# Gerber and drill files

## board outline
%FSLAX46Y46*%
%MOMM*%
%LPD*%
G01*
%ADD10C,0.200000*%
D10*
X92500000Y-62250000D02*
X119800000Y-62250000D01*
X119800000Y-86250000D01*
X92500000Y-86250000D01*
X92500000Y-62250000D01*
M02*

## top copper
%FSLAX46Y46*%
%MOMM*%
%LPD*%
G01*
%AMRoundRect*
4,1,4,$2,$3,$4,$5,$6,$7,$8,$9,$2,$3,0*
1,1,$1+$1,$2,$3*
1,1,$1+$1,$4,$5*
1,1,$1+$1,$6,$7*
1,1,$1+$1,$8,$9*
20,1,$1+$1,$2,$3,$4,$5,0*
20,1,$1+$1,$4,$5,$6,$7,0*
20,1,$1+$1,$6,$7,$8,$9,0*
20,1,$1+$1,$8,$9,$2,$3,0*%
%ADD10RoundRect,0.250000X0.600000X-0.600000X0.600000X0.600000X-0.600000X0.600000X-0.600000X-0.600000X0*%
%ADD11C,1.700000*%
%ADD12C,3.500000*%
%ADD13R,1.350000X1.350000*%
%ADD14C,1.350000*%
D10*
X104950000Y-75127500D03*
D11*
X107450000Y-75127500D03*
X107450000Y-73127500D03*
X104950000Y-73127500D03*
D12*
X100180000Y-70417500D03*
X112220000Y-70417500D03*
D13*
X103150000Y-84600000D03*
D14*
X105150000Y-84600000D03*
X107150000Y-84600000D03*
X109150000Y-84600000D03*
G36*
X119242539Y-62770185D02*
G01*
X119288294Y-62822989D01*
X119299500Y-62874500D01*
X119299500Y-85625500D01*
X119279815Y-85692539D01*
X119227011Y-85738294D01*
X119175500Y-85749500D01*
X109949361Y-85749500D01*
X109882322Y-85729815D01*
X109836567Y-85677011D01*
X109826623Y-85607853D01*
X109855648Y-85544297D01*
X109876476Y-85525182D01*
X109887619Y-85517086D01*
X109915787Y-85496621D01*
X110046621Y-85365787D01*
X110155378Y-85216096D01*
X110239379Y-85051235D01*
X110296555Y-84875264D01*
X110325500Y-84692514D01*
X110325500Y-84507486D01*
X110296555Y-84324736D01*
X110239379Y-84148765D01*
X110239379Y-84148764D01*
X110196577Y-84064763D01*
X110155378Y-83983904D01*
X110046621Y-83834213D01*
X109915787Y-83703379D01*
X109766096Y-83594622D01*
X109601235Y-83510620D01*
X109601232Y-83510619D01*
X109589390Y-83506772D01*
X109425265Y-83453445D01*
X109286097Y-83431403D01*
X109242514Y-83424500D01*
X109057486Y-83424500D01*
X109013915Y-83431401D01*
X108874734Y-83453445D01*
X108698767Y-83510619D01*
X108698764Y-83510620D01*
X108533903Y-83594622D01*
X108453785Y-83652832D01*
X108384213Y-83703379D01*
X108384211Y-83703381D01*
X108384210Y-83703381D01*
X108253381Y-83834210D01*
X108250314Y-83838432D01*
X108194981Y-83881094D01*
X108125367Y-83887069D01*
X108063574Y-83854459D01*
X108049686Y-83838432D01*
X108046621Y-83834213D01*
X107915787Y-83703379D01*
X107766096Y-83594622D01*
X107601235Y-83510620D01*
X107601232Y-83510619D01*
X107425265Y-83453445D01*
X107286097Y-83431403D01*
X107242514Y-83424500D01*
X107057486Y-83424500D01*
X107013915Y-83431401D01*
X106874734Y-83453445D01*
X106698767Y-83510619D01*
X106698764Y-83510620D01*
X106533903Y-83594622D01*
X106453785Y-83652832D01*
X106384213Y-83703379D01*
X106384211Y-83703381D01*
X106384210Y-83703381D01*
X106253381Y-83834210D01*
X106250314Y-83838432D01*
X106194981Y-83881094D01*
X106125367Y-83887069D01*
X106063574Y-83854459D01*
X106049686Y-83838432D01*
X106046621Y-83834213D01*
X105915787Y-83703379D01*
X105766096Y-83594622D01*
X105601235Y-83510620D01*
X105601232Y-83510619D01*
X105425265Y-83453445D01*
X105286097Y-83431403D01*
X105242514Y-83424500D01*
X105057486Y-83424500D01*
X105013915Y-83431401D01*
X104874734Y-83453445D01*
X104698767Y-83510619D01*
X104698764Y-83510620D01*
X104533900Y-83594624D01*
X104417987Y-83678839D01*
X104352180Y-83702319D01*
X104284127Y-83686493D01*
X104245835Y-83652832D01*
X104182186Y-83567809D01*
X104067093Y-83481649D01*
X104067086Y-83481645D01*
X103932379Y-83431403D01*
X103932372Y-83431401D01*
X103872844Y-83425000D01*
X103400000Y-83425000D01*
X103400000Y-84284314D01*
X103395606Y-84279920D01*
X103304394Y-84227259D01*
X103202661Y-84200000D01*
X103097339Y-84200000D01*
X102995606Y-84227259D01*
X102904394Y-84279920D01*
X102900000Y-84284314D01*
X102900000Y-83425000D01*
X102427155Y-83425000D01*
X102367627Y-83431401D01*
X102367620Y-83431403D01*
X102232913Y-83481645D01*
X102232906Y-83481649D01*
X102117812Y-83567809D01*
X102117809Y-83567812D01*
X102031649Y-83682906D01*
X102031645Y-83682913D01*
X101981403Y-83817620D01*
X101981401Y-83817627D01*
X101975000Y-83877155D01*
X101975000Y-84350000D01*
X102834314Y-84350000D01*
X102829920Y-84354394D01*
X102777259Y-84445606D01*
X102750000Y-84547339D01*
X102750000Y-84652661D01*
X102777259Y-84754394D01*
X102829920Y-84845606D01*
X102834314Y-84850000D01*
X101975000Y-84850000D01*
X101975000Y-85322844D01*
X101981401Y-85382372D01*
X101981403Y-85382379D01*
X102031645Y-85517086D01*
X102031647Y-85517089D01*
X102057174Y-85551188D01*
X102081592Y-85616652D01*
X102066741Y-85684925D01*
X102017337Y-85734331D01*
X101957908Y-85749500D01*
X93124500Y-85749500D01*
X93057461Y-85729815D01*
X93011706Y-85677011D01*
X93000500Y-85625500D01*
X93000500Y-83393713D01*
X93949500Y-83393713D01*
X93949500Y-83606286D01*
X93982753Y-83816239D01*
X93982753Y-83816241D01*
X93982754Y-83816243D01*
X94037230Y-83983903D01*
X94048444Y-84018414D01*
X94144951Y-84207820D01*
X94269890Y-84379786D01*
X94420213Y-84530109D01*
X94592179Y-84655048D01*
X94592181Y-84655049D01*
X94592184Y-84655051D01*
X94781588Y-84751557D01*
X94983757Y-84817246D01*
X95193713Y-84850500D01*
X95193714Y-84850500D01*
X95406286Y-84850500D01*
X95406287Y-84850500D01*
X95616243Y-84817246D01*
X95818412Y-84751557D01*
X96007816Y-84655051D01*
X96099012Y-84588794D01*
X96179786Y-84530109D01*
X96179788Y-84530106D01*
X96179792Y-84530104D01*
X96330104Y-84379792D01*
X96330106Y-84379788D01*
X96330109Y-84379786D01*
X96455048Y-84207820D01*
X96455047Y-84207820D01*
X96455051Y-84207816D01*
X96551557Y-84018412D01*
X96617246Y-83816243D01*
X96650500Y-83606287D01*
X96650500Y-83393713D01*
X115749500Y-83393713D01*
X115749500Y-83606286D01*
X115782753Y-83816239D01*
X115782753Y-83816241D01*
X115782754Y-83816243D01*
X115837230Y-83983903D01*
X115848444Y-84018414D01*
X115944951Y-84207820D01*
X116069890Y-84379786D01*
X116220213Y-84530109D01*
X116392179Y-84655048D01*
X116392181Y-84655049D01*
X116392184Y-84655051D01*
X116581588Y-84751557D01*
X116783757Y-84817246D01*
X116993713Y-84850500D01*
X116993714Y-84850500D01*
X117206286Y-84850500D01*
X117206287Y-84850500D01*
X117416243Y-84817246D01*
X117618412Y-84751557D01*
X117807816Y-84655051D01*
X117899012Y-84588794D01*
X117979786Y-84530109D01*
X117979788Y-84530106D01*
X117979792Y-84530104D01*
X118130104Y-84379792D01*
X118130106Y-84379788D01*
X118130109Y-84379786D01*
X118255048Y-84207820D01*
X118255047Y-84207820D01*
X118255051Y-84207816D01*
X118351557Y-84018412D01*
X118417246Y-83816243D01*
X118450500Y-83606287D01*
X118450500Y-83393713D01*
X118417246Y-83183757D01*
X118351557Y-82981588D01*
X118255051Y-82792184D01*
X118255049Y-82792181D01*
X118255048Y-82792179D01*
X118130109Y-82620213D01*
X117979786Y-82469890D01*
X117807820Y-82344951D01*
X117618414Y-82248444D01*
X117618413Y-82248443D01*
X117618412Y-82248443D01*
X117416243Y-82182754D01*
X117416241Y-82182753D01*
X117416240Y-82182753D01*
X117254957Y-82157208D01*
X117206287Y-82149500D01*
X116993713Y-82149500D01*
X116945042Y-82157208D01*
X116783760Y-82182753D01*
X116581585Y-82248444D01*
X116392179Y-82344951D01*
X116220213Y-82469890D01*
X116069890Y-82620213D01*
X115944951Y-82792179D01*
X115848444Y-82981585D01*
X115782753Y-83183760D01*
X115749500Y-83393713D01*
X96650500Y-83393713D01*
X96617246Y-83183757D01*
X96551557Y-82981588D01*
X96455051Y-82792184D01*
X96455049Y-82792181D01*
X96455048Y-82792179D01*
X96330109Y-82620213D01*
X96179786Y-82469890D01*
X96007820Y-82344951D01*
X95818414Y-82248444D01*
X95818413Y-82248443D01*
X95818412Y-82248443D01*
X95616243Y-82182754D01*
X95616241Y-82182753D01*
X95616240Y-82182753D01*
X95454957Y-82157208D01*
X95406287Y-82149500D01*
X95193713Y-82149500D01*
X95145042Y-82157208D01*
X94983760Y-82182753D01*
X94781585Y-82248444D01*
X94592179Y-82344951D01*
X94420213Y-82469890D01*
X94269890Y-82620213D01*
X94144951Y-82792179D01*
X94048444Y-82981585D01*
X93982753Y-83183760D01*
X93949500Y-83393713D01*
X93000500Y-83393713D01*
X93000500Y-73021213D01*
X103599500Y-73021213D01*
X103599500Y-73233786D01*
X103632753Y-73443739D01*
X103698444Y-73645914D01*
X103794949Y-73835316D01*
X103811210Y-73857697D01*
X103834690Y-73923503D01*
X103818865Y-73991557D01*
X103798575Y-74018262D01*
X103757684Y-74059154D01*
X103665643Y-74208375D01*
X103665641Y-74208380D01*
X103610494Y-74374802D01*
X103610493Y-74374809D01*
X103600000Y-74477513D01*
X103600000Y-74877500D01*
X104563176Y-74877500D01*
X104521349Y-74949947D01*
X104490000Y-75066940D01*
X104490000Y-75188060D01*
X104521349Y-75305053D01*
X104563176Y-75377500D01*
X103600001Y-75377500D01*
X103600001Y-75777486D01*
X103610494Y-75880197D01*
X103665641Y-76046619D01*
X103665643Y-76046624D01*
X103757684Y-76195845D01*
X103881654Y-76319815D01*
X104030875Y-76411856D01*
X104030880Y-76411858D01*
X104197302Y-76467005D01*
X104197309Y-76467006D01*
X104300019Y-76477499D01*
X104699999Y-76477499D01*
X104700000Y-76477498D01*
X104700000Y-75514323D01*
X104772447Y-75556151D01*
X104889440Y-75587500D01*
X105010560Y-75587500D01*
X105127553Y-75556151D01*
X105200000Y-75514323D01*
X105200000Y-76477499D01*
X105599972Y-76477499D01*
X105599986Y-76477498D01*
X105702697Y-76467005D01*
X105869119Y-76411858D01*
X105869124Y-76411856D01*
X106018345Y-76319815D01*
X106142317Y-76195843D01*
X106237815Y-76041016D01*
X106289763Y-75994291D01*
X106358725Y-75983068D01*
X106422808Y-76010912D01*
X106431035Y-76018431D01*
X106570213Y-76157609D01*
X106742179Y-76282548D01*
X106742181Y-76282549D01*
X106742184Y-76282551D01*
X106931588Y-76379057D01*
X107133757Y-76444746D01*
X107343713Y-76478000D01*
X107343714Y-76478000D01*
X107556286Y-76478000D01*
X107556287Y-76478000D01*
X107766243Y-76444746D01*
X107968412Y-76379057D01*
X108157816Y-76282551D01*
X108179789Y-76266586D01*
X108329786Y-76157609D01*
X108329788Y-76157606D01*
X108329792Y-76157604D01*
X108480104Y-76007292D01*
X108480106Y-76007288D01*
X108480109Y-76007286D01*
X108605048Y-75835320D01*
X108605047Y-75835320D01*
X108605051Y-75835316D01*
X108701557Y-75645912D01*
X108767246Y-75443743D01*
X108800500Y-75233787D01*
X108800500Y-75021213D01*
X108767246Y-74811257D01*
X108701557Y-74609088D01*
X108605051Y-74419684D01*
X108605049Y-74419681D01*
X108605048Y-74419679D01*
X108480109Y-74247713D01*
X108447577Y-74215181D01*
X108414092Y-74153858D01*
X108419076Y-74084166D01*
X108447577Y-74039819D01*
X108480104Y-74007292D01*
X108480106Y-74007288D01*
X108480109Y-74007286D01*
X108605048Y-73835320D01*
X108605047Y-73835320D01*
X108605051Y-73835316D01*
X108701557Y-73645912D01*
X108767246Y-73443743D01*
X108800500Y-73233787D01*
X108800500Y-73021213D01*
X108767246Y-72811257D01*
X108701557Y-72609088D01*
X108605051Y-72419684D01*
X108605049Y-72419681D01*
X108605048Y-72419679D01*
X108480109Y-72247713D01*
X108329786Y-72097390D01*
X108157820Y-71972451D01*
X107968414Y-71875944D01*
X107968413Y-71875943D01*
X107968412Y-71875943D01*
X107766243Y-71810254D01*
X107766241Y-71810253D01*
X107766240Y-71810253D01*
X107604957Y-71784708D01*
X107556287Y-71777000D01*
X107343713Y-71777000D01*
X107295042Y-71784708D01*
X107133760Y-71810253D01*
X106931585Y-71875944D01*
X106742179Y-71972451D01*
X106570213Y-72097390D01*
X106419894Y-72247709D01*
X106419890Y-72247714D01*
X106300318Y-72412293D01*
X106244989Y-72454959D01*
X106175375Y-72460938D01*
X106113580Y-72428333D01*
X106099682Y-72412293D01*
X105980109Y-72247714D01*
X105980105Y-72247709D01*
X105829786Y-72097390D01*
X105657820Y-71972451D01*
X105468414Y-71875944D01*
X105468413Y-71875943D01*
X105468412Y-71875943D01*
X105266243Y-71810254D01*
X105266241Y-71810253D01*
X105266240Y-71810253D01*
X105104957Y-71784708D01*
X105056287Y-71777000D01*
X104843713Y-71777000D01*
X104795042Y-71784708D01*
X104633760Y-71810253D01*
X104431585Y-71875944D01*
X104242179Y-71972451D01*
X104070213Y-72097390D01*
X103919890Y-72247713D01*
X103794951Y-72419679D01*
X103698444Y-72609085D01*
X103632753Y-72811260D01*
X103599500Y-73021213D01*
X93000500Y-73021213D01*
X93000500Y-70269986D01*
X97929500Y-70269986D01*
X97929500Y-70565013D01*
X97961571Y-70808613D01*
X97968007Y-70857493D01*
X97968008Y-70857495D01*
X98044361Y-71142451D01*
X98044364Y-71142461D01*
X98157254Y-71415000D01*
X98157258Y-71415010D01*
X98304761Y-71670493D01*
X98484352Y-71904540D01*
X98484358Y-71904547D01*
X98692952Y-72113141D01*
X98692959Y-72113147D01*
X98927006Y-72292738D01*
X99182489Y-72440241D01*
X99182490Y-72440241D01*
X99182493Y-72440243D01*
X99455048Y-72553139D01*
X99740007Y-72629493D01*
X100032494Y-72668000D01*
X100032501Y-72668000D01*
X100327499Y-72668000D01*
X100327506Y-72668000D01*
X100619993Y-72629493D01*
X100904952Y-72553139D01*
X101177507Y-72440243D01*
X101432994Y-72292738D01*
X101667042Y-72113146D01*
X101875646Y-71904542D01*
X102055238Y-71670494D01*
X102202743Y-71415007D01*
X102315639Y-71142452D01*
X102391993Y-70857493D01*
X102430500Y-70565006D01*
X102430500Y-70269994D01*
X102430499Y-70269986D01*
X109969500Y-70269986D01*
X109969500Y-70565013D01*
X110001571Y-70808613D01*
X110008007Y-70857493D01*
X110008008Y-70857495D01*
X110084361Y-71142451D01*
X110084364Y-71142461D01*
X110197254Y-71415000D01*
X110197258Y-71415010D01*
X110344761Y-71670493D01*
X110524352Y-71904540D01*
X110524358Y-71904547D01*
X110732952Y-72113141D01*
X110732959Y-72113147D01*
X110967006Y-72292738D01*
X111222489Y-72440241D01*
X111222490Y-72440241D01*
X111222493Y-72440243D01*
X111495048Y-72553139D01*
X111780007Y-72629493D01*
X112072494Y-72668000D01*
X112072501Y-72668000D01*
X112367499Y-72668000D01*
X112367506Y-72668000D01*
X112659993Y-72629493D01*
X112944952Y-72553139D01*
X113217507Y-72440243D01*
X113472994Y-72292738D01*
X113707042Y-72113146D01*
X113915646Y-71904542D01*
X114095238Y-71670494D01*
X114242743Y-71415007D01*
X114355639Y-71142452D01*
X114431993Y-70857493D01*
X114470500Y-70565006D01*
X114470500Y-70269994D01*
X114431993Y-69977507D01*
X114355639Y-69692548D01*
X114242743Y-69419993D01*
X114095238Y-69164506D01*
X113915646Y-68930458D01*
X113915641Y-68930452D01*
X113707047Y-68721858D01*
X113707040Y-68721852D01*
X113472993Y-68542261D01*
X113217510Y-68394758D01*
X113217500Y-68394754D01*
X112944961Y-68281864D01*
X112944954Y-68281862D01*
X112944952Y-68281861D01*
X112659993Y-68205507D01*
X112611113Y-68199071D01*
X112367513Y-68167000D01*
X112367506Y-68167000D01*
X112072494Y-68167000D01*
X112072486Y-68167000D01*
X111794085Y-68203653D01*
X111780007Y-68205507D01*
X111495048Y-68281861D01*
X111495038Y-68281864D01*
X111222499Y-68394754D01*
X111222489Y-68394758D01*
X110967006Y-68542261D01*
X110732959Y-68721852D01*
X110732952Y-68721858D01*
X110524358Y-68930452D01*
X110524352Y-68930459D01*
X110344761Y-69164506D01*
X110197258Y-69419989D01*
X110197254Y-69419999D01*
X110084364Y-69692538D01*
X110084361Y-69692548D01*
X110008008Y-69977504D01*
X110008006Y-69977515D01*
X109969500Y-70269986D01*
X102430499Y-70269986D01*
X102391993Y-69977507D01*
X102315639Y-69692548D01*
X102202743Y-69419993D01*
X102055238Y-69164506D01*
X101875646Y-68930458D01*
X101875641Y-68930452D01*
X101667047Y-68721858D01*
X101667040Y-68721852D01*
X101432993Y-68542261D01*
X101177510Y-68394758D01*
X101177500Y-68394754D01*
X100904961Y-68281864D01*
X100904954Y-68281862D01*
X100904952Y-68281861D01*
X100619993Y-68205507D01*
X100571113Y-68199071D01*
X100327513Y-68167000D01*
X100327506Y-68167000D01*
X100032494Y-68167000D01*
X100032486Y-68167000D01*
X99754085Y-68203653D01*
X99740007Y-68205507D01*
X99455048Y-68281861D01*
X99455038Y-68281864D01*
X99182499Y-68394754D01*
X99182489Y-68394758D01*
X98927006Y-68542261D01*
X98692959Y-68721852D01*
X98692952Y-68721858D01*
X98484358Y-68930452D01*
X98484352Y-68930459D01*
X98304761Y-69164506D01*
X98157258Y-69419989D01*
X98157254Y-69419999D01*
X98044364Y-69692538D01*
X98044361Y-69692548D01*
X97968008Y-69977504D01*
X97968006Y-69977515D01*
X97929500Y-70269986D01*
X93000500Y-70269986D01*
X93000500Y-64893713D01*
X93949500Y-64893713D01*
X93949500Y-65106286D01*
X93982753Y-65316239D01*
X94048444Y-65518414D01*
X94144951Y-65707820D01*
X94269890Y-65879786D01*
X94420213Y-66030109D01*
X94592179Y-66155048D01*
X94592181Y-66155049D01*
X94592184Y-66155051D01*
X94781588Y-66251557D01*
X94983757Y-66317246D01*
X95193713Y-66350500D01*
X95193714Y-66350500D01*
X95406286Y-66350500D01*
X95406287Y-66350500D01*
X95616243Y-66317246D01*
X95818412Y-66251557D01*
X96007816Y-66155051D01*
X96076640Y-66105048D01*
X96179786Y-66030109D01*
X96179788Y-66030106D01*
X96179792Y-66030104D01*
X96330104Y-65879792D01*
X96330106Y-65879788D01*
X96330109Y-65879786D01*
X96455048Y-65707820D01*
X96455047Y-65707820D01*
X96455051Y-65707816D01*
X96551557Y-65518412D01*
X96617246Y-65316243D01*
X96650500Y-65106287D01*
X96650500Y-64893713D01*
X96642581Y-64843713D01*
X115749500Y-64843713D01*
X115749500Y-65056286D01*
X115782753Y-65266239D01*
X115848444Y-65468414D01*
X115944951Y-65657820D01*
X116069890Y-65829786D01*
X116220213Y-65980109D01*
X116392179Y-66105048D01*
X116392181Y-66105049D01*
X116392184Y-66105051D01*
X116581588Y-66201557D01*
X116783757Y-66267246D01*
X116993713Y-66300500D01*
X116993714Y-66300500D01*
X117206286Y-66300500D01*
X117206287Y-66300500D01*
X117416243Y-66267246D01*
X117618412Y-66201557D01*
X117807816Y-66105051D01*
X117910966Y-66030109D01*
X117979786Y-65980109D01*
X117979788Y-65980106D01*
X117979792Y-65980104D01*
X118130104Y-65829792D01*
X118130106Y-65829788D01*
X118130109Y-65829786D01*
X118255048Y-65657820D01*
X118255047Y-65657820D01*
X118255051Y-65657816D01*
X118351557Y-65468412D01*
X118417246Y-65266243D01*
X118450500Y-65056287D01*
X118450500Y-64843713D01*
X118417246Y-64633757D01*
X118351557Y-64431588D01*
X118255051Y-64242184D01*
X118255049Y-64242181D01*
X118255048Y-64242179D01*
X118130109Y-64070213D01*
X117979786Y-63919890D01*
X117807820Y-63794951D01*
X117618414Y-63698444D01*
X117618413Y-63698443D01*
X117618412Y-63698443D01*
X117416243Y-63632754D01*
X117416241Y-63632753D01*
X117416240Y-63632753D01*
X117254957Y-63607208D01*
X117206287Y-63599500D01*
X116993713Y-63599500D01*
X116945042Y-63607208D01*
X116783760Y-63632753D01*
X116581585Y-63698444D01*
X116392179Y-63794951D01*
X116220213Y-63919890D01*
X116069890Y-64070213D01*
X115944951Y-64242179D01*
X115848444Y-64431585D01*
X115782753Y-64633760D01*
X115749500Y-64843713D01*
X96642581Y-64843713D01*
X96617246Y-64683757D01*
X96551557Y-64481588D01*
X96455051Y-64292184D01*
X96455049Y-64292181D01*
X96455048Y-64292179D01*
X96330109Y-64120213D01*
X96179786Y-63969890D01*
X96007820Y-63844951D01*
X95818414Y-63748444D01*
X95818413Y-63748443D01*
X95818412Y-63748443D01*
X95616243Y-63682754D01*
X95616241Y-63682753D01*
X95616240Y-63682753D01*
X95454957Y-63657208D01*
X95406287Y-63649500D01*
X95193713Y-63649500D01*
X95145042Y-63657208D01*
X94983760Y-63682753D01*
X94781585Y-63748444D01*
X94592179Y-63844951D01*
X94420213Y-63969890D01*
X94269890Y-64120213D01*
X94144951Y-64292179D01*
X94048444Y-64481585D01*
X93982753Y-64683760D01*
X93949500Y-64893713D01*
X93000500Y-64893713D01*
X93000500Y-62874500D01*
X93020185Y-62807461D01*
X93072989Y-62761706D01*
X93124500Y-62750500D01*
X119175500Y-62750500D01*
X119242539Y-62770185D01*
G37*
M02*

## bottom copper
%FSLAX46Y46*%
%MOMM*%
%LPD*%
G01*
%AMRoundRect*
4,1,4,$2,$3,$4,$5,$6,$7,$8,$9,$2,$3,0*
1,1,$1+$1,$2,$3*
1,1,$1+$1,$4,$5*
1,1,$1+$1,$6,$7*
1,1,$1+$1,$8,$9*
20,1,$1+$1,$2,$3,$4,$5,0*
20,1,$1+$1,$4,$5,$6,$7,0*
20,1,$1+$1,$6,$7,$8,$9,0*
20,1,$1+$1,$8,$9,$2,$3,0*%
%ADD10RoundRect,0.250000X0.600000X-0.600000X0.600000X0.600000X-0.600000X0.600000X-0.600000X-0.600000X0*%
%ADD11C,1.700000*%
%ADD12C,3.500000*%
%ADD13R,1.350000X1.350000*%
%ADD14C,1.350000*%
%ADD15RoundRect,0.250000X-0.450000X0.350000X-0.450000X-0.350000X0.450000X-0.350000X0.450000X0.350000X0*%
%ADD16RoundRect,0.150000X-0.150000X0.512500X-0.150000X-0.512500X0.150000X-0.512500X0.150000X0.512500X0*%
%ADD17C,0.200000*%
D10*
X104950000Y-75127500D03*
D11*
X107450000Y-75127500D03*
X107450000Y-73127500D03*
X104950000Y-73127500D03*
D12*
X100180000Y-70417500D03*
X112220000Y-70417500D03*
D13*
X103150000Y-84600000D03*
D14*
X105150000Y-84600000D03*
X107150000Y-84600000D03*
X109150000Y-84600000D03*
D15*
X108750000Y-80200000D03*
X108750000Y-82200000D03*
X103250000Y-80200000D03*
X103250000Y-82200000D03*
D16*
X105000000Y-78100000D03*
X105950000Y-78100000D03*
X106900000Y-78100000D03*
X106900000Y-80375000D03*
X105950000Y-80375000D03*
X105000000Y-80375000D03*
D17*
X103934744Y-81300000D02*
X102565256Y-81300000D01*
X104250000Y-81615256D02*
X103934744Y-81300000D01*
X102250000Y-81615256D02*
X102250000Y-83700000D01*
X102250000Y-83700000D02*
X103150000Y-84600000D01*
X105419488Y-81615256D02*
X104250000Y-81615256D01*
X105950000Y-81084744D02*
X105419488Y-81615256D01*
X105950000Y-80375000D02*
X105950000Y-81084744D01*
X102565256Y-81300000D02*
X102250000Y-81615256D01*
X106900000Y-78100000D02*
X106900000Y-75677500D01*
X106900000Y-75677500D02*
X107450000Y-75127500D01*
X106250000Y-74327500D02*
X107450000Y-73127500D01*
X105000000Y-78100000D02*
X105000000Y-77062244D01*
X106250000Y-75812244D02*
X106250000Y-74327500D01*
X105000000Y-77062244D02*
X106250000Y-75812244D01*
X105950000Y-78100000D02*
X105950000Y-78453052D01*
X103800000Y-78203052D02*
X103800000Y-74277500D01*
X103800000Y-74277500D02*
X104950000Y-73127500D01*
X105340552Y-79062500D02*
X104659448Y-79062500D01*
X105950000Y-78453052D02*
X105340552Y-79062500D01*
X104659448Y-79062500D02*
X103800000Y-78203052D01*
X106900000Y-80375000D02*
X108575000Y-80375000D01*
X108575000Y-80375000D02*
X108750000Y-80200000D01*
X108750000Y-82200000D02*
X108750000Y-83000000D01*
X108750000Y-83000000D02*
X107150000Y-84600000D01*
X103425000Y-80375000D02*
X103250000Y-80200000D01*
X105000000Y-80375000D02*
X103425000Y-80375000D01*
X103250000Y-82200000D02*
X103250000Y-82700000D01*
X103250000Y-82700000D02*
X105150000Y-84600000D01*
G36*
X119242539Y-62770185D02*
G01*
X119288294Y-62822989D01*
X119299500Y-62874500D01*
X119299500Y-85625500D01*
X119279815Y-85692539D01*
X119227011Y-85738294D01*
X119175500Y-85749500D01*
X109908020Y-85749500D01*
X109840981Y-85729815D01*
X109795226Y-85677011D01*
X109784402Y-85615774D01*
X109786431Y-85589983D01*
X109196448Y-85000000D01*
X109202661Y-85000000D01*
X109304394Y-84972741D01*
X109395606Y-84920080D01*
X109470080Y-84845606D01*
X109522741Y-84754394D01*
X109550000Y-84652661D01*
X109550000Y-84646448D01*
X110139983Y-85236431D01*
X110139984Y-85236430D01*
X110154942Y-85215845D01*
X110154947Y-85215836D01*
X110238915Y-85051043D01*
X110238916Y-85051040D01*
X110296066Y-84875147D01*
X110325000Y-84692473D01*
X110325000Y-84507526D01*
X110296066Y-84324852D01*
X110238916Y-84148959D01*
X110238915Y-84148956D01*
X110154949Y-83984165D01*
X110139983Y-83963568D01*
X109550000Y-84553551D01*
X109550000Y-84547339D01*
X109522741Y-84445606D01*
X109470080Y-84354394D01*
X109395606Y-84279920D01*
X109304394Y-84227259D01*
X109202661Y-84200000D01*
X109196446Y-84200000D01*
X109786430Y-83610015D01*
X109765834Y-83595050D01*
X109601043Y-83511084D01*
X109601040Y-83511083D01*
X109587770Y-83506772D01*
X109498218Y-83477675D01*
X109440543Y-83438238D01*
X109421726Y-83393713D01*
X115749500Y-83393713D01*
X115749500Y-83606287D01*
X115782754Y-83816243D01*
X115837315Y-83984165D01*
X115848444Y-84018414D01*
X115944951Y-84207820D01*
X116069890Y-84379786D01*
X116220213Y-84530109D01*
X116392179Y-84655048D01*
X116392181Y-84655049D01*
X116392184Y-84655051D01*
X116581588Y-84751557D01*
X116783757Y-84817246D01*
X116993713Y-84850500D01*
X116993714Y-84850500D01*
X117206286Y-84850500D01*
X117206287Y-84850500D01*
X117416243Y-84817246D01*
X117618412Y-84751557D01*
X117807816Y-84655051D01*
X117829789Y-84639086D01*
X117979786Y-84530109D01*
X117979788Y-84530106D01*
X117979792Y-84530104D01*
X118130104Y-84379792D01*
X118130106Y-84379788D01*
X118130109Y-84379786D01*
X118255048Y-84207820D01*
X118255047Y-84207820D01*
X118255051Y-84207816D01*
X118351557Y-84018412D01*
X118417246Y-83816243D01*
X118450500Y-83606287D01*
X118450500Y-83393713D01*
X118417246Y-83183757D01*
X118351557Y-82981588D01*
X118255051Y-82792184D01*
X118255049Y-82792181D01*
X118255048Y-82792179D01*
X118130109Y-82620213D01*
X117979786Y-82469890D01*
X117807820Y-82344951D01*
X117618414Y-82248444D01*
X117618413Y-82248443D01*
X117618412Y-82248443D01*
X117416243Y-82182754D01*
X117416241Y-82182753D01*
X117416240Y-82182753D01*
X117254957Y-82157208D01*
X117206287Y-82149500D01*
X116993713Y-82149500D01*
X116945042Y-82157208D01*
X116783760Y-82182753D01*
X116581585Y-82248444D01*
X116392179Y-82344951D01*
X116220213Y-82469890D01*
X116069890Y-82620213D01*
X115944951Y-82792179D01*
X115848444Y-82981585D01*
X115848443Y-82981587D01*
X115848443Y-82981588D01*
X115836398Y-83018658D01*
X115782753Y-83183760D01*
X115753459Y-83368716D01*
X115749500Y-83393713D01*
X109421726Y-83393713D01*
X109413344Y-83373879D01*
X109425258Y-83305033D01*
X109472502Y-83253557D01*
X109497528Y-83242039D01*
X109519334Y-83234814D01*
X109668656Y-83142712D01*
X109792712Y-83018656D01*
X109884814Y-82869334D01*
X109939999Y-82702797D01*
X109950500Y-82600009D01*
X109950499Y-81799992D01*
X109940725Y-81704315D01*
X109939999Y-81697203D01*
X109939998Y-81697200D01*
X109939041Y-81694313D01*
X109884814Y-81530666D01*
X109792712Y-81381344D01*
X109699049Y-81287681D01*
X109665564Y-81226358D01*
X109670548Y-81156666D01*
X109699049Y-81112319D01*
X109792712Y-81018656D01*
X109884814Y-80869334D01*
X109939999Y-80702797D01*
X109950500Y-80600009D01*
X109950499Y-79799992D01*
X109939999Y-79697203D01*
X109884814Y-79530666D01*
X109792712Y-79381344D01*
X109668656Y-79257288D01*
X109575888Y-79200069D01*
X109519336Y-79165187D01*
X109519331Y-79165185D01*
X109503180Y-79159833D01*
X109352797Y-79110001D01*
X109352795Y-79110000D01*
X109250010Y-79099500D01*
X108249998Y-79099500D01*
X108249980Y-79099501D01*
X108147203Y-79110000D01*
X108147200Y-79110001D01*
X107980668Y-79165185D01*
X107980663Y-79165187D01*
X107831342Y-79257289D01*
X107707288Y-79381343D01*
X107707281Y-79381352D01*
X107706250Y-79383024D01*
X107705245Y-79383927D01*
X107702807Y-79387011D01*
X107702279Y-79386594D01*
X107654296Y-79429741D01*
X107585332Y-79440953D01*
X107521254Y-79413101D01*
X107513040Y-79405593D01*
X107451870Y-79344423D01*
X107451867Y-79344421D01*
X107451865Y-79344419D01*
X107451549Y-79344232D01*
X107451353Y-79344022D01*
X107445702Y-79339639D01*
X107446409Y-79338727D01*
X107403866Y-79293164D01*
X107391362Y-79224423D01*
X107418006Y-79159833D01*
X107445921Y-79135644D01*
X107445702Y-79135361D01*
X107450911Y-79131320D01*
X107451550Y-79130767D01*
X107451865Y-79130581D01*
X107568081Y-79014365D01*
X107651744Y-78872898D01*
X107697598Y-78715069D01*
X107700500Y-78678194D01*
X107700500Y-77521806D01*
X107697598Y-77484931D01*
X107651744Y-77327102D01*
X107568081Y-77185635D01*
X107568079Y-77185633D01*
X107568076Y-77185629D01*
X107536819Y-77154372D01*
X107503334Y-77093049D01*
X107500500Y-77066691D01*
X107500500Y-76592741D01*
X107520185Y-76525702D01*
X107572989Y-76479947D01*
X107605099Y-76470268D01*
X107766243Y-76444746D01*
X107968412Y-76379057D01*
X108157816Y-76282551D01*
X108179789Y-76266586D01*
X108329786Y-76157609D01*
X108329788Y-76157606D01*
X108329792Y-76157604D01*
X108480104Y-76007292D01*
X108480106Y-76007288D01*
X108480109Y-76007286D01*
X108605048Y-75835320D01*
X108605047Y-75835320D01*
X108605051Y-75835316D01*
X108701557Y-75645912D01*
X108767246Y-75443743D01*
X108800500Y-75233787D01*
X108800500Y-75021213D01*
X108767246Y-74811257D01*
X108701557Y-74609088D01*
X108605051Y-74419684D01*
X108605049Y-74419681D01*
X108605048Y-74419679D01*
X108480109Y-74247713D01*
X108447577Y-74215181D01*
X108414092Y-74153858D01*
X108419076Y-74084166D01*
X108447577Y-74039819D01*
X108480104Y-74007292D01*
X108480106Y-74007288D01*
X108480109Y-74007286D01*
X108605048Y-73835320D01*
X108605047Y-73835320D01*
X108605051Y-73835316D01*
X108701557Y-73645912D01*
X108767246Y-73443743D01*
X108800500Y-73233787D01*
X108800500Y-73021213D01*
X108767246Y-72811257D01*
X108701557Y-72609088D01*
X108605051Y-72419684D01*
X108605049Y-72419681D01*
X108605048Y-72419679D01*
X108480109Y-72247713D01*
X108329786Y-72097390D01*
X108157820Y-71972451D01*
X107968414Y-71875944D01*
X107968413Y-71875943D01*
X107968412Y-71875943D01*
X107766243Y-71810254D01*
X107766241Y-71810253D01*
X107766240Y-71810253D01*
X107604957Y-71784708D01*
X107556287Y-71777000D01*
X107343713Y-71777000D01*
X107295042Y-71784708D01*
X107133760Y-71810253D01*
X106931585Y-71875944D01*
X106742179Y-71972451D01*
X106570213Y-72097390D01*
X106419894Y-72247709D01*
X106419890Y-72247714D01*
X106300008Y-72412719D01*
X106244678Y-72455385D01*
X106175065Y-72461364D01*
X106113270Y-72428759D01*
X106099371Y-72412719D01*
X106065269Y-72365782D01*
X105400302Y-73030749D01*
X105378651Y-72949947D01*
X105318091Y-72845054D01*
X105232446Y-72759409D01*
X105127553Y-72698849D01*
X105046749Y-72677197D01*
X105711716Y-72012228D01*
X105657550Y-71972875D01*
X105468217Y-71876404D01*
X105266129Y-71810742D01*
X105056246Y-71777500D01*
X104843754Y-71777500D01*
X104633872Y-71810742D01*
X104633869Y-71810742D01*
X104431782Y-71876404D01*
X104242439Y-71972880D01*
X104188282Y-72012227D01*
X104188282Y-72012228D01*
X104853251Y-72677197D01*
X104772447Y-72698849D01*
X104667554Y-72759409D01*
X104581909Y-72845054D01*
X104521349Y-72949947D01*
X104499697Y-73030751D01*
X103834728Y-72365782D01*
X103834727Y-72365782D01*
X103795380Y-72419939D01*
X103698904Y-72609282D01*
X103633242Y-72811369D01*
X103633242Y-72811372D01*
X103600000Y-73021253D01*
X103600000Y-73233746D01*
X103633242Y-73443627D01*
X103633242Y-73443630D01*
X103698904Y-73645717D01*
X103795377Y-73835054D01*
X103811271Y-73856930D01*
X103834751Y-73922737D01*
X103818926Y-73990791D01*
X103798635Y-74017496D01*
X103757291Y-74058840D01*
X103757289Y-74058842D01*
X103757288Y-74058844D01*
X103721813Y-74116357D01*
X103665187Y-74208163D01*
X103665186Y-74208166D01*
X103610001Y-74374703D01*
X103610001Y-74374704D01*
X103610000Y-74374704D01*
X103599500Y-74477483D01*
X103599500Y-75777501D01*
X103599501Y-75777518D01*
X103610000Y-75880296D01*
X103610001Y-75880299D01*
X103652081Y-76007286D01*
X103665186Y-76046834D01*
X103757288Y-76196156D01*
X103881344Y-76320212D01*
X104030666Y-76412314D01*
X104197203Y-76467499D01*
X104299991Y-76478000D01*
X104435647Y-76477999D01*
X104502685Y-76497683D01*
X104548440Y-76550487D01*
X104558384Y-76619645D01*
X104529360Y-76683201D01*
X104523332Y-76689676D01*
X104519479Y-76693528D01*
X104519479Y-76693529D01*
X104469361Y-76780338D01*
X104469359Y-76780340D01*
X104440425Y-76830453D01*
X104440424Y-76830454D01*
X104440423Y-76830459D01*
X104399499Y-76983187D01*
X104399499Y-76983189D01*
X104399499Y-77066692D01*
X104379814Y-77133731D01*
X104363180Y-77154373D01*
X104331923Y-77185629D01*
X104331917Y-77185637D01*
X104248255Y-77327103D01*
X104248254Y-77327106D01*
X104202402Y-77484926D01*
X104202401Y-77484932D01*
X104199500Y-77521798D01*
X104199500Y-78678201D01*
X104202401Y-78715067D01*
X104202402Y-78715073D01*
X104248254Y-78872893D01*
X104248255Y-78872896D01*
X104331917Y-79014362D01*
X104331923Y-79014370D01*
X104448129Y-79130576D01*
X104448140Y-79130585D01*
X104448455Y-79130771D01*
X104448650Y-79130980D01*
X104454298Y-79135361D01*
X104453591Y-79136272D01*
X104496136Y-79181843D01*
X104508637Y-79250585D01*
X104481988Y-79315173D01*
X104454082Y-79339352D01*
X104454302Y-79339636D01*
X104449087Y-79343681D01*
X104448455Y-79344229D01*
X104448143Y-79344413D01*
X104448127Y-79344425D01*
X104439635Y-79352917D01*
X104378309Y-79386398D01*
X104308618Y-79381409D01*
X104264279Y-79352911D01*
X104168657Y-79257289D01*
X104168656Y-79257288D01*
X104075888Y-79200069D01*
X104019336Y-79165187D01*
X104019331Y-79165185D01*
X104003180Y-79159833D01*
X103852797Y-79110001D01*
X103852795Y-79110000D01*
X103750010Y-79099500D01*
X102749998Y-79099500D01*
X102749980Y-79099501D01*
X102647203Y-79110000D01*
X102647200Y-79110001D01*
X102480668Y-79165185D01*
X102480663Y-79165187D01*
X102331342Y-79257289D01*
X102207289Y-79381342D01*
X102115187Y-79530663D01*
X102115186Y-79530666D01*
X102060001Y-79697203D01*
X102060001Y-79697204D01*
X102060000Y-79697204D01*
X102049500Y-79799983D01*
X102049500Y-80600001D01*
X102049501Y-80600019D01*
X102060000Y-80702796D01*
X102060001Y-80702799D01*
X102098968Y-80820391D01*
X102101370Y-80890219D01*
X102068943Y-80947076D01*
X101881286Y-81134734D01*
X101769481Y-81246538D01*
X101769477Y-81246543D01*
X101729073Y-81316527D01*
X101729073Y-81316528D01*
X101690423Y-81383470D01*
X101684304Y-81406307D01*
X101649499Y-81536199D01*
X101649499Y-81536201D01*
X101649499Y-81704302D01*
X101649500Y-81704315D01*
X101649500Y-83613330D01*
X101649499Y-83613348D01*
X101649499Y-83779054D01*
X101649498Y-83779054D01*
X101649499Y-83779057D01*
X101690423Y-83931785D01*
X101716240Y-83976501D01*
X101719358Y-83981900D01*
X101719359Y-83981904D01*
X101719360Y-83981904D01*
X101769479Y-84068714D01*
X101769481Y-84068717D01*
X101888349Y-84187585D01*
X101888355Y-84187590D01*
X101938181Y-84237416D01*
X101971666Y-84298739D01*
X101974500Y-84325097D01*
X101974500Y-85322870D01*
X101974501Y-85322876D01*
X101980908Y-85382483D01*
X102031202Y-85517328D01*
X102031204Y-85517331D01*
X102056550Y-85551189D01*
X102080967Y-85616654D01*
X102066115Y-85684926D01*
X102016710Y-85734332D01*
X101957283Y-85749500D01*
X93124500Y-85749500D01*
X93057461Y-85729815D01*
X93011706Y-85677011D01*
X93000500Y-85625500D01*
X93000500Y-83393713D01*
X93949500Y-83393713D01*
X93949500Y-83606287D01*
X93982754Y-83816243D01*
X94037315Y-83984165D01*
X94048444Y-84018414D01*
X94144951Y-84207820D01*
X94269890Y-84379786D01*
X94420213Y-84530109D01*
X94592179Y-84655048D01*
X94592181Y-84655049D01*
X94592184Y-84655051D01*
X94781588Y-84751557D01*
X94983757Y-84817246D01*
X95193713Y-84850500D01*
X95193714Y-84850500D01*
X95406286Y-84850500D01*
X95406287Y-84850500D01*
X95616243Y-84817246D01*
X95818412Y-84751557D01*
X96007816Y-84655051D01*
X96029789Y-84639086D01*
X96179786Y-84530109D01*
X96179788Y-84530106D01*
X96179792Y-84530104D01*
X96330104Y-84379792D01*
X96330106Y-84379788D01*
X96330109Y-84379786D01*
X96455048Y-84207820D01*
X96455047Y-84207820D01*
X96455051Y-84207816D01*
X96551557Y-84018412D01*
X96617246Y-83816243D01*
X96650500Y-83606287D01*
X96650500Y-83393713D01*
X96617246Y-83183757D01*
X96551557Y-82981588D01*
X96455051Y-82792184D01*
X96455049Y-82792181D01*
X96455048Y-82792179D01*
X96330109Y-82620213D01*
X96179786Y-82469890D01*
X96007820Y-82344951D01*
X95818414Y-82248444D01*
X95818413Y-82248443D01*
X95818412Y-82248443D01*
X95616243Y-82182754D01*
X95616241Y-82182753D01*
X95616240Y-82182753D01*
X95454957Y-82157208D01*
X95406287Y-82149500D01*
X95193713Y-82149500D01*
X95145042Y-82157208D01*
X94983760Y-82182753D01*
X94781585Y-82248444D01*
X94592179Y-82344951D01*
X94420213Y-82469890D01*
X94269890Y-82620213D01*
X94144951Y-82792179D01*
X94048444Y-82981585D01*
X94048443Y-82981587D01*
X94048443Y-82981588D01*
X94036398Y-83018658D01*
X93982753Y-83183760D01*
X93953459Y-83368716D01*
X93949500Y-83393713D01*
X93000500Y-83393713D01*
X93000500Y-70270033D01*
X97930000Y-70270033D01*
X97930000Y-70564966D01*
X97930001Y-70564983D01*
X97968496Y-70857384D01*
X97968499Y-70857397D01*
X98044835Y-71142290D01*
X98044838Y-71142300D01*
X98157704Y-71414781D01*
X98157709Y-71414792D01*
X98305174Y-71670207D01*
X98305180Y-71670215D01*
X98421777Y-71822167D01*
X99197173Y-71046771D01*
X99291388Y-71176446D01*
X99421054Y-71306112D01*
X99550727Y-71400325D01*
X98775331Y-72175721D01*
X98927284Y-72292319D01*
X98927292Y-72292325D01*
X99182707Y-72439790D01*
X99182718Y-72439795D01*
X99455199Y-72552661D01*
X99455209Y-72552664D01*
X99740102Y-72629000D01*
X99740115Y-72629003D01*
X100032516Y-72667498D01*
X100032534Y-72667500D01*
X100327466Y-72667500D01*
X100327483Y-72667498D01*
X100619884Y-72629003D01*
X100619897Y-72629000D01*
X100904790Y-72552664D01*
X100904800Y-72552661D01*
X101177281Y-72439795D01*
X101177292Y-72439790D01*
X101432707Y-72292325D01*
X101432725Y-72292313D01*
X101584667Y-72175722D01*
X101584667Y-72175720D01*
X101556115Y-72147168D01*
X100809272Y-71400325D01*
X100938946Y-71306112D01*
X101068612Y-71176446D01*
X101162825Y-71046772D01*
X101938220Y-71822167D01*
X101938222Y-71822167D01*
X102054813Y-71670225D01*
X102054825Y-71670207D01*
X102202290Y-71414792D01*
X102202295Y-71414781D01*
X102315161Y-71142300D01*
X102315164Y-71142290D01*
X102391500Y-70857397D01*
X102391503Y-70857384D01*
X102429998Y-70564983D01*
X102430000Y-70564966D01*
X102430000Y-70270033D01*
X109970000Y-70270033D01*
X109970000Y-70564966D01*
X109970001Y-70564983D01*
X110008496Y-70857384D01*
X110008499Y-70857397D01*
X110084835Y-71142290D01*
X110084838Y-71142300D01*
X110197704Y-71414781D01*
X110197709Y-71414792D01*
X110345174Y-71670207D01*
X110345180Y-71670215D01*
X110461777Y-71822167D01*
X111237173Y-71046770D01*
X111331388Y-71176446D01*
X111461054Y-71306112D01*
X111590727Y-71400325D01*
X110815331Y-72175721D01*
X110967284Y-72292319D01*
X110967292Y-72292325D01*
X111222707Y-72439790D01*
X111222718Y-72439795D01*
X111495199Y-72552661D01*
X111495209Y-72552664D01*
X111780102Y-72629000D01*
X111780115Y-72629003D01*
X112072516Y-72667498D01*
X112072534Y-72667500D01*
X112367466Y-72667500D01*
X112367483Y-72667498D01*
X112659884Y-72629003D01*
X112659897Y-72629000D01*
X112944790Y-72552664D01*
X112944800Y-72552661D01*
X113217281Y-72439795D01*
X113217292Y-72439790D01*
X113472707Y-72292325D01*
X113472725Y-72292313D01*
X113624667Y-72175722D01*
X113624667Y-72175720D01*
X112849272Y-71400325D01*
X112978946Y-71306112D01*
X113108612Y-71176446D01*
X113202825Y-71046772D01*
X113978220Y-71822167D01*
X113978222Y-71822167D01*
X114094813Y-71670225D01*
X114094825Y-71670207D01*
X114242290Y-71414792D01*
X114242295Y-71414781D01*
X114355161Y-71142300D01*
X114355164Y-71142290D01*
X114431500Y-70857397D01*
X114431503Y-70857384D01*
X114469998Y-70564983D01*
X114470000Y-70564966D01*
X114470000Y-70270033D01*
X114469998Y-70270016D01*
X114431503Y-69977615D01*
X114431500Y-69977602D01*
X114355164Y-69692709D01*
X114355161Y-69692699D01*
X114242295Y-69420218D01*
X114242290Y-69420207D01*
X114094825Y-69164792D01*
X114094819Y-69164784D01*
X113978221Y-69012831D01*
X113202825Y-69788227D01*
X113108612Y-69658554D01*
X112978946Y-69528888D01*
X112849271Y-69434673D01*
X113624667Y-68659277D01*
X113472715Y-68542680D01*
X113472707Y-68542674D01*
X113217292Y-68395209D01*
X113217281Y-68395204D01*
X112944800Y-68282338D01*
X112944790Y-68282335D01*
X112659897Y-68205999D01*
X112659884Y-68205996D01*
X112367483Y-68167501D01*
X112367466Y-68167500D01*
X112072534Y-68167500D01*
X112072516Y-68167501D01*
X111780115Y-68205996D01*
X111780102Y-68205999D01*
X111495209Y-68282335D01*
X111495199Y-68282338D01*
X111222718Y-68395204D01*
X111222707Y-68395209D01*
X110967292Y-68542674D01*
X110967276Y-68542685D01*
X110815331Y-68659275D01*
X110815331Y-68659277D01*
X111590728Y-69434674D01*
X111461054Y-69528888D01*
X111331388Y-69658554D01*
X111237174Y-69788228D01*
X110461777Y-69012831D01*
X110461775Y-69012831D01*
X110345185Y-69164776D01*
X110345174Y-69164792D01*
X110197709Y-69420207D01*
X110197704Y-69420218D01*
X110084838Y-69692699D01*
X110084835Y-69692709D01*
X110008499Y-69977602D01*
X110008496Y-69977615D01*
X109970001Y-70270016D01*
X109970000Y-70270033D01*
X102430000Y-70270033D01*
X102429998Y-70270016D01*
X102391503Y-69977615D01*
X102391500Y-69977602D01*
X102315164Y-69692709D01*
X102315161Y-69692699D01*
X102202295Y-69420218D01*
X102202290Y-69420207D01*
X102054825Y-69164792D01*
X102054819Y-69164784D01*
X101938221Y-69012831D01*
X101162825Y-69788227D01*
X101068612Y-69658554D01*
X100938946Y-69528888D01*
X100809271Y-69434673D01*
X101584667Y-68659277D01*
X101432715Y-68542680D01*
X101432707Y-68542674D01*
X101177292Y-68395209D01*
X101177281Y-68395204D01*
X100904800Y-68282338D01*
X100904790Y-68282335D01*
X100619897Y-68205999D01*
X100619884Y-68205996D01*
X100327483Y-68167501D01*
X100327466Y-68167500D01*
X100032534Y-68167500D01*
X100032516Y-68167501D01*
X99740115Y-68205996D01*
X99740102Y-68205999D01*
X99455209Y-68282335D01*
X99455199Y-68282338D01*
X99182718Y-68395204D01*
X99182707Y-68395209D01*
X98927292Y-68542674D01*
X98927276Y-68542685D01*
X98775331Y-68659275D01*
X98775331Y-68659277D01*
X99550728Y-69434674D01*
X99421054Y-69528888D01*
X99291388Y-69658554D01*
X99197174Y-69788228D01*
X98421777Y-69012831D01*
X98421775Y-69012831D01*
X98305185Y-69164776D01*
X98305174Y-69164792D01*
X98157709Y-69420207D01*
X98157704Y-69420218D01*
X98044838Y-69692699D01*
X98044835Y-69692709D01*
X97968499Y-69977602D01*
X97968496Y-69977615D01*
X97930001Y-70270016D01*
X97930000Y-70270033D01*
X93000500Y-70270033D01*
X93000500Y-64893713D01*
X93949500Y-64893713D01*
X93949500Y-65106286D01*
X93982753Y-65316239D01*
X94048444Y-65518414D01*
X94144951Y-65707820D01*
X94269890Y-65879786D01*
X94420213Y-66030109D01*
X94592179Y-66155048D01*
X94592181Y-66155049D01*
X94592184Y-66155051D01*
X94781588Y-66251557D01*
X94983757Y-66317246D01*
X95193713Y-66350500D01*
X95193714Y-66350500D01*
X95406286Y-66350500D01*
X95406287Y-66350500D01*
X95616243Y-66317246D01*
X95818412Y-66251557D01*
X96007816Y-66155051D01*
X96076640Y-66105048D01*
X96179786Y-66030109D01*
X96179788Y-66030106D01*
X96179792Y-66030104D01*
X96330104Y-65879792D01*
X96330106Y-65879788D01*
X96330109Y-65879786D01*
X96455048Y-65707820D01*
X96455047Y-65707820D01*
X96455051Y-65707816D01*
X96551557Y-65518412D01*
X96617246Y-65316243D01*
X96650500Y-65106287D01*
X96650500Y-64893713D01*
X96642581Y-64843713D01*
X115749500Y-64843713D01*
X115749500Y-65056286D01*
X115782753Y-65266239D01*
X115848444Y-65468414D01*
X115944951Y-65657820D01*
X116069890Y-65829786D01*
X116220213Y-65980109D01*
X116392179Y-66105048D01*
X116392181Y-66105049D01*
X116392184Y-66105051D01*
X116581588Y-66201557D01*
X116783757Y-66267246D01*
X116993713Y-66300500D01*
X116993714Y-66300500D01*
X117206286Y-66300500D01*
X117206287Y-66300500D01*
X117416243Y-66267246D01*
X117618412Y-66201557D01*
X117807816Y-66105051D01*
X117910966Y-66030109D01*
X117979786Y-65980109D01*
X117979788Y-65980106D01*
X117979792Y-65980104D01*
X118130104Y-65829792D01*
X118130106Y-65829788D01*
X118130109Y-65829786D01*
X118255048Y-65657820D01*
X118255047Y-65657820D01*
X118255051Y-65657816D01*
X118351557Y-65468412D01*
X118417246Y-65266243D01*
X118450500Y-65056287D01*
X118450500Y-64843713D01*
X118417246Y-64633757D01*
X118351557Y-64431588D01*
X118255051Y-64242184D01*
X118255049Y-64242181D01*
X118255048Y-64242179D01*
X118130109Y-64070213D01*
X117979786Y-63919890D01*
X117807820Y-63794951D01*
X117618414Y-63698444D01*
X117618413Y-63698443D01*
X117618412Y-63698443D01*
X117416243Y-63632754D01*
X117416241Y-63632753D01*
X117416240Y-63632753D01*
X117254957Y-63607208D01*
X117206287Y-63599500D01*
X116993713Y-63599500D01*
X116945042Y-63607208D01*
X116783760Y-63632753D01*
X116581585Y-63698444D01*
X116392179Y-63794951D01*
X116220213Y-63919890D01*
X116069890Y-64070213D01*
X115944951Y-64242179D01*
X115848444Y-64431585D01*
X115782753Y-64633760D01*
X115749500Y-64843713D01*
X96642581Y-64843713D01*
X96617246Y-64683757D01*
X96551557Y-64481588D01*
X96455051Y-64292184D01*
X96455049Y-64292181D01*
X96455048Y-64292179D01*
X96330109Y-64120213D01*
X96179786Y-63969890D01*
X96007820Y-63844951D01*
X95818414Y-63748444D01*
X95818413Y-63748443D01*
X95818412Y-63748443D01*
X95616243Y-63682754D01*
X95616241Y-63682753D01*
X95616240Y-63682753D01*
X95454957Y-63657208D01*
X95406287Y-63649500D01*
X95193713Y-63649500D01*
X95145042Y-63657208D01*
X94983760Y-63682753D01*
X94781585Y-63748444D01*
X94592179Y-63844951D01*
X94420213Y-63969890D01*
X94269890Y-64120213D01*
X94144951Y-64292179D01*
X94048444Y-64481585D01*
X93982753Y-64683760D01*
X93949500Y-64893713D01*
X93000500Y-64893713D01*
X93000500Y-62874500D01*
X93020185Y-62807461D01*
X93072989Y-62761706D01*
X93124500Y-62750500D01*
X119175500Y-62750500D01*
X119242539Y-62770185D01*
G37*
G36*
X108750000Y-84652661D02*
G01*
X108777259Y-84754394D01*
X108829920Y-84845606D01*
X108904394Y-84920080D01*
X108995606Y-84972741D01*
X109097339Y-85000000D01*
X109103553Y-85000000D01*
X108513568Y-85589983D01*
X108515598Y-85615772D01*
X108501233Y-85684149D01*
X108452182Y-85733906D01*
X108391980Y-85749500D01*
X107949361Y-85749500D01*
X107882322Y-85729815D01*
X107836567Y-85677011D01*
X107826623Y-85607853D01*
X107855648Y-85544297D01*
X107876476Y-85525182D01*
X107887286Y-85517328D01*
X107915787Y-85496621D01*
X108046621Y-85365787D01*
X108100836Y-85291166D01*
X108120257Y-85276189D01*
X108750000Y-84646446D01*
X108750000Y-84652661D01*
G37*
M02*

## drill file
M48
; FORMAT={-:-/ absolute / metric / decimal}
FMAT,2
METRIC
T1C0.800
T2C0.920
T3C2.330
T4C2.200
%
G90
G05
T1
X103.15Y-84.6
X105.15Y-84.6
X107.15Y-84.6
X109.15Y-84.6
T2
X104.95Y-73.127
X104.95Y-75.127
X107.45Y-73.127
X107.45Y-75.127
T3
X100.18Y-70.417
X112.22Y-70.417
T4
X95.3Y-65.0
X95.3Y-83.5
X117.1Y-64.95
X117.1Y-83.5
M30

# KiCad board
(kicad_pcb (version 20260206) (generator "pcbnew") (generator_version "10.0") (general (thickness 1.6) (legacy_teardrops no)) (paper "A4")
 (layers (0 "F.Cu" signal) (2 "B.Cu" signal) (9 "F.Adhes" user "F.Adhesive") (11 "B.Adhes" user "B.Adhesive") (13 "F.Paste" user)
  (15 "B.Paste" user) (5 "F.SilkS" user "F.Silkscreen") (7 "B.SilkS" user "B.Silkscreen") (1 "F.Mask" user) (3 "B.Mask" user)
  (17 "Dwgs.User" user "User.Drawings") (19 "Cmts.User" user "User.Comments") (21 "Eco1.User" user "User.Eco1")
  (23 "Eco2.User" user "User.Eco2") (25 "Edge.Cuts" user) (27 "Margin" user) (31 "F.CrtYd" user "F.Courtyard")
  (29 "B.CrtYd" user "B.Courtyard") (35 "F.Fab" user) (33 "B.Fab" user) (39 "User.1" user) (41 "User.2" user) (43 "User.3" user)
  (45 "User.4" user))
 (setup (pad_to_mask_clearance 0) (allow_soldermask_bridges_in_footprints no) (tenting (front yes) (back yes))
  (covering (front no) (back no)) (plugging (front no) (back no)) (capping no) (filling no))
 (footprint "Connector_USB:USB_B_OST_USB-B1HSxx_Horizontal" (layer "F.Cu") (at 104.95 75.1275 90)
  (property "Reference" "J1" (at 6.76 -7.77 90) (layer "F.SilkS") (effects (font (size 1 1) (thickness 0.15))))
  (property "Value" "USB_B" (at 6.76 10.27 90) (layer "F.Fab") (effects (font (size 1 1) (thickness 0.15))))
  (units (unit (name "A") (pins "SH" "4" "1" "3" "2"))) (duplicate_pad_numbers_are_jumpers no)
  (pad "1" thru_hole roundrect (at 0 0 90) (size 1.7 1.7) (drill 0.92) (layers "*.Cu" "*.Mask") (remove_unused_layers no)
   (roundrect_rratio 0.1470588235) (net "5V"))
  (pad "2" thru_hole circle (at 0 2.5 90) (size 1.7 1.7) (drill 0.92) (layers "*.Cu" "*.Mask") (remove_unused_layers no) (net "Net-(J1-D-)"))
  (pad "3" thru_hole circle (at 2 2.5 90) (size 1.7 1.7) (drill 0.92) (layers "*.Cu" "*.Mask") (remove_unused_layers no) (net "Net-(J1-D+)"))
  (pad "4" thru_hole circle (at 2 0 90) (size 1.7 1.7) (drill 0.92) (layers "*.Cu" "*.Mask") (remove_unused_layers no) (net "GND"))
  (pad "SH" thru_hole circle (at 4.71 -4.77 90) (size 3.5 3.5) (drill 2.33) (layers "*.Cu" "*.Mask") (remove_unused_layers no) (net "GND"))
  (pad "SH" thru_hole circle (at 4.71 7.27 90) (size 3.5 3.5) (drill 2.33) (layers "*.Cu" "*.Mask") (remove_unused_layers no) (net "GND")))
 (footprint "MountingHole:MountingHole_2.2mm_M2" (layer "F.Cu") (at 117.1 83.5)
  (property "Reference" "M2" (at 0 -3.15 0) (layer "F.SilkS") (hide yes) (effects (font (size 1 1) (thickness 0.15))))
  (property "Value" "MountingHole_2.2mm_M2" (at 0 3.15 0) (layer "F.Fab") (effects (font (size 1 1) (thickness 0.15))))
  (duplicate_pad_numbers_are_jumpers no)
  (pad "" np_thru_hole circle (at 0 0) (size 2.2 2.2) (drill 2.2) (layers "*.Cu" "*.Mask")))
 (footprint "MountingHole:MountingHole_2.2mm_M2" (layer "F.Cu") (at 95.3 65)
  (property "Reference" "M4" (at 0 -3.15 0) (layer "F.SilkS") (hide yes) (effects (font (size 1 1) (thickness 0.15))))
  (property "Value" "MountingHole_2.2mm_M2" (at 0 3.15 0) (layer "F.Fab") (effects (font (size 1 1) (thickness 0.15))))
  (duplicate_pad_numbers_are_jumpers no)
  (pad "" np_thru_hole circle (at 0 0) (size 2.2 2.2) (drill 2.2) (layers "*.Cu" "*.Mask")))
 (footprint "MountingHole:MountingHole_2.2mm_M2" (layer "F.Cu") (at 117.1 64.95)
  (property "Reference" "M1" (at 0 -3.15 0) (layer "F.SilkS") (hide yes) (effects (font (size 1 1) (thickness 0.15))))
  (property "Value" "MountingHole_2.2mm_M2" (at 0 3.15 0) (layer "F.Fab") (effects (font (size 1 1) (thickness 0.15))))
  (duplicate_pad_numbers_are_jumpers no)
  (pad "" np_thru_hole circle (at 0 0) (size 2.2 2.2) (drill 2.2) (layers "*.Cu" "*.Mask")))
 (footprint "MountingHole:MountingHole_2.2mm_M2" (layer "F.Cu") (at 95.3 83.5)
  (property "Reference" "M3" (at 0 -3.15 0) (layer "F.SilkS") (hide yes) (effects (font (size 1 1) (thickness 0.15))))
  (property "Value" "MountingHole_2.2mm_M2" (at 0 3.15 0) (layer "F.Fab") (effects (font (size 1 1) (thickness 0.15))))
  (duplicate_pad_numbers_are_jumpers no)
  (pad "" np_thru_hole circle (at 0 0) (size 2.2 2.2) (drill 2.2) (layers "*.Cu" "*.Mask")))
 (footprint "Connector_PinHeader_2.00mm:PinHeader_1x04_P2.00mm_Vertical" (layer "F.Cu") (at 103.15 84.6 90)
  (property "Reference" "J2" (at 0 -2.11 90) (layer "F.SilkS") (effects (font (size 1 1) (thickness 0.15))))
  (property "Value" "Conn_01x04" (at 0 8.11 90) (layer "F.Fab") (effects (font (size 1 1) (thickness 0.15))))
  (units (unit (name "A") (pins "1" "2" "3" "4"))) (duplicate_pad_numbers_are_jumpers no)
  (pad "1" thru_hole rect (at 0 0 90) (size 1.35 1.35) (drill 0.8) (layers "*.Cu" "*.Mask") (remove_unused_layers no) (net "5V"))
  (pad "2" thru_hole circle (at 0 2 90) (size 1.35 1.35) (drill 0.8) (layers "*.Cu" "*.Mask") (remove_unused_layers no)
   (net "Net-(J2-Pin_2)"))
  (pad "3" thru_hole circle (at 0 4 90) (size 1.35 1.35) (drill 0.8) (layers "*.Cu" "*.Mask") (remove_unused_layers no)
   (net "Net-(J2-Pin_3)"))
  (pad "4" thru_hole circle (at 0 6 90) (size 1.35 1.35) (drill 0.8) (layers "*.Cu" "*.Mask") (remove_unused_layers no) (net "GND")))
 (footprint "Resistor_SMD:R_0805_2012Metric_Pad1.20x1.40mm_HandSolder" (layer "B.Cu") (at 108.75 81.2 -90)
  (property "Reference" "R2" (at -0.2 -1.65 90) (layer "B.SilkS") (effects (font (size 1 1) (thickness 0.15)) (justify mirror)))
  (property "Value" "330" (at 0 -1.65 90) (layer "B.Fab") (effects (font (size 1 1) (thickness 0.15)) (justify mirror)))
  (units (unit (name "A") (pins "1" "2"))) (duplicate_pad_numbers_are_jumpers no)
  (pad "1" smd roundrect (at -1 0 270) (size 1.2 1.4) (layers "B.Cu" "B.Mask" "B.Paste") (roundrect_rratio 0.208333) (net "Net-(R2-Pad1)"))
  (pad "2" smd roundrect (at 1 0 270) (size 1.2 1.4) (layers "B.Cu" "B.Mask" "B.Paste") (roundrect_rratio 0.208333) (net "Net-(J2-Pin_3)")))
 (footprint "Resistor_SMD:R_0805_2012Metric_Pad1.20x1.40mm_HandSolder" (layer "B.Cu") (at 103.25 81.2 -90)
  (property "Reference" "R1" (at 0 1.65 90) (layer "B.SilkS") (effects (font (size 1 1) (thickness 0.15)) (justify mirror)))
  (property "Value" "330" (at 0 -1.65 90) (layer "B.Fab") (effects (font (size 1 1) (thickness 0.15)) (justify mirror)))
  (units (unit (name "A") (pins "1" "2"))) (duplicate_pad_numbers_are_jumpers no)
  (pad "1" smd roundrect (at -1 0 270) (size 1.2 1.4) (layers "B.Cu" "B.Mask" "B.Paste") (roundrect_rratio 0.208333) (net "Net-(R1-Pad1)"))
  (pad "2" smd roundrect (at 1 0 270) (size 1.2 1.4) (layers "B.Cu" "B.Mask" "B.Paste") (roundrect_rratio 0.208333) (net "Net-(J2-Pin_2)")))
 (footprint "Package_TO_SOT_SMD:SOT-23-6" (layer "B.Cu") (at 105.95 79.2375 -90)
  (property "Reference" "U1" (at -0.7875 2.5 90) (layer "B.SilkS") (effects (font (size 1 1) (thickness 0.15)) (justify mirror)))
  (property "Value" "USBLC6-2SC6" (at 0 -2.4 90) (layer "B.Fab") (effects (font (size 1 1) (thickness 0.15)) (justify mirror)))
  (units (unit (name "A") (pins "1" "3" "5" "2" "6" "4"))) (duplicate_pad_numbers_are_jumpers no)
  (pad "1" smd roundrect (at -1.1375 0.95 270) (size 1.325 0.6) (layers "B.Cu" "B.Mask" "B.Paste") (roundrect_rratio 0.25)
   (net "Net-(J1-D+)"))
  (pad "2" smd roundrect (at -1.1375 0 270) (size 1.325 0.6) (layers "B.Cu" "B.Mask" "B.Paste") (roundrect_rratio 0.25) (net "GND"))
  (pad "3" smd roundrect (at -1.1375 -0.95 270) (size 1.325 0.6) (layers "B.Cu" "B.Mask" "B.Paste") (roundrect_rratio 0.25)
   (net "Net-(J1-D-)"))
  (pad "4" smd roundrect (at 1.1375 -0.95 270) (size 1.325 0.6) (layers "B.Cu" "B.Mask" "B.Paste") (roundrect_rratio 0.25)
   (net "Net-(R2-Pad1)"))
  (pad "5" smd roundrect (at 1.1375 0 270) (size 1.325 0.6) (layers "B.Cu" "B.Mask" "B.Paste") (roundrect_rratio 0.25) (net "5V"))
  (pad "6" smd roundrect (at 1.1375 0.95 270) (size 1.325 0.6) (layers "B.Cu" "B.Mask" "B.Paste") (roundrect_rratio 0.25)
   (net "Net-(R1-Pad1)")))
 (gr_rect (start 92.5 62.25) (end 119.8 86.25) (stroke (width 0.2) (type solid)) (fill no) (layer "Edge.Cuts"))
 (segment (start 103.934744 81.3) (end 102.565256 81.3) (width 0.2) (layer "B.Cu") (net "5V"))
 (segment (start 104.25 81.615256) (end 103.934744 81.3) (width 0.2) (layer "B.Cu") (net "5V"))
 (segment (start 102.25 81.615256) (end 102.25 83.7) (width 0.2) (layer "B.Cu") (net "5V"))
 (segment (start 102.25 83.7) (end 103.15 84.6) (width 0.2) (layer "B.Cu") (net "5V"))
 (segment (start 105.419488 81.615256) (end 104.25 81.615256) (width 0.2) (layer "B.Cu") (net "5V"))
 (segment (start 105.95 81.084744) (end 105.419488 81.615256) (width 0.2) (layer "B.Cu") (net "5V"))
 (segment (start 105.95 80.375) (end 105.95 81.084744) (width 0.2) (layer "B.Cu") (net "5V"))
 (segment (start 102.565256 81.3) (end 102.25 81.615256) (width 0.2) (layer "B.Cu") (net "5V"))
 (segment (start 106.9 78.1) (end 106.9 75.6775) (width 0.2) (layer "B.Cu") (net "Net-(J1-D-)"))
 (segment (start 106.9 75.6775) (end 107.45 75.1275) (width 0.2) (layer "B.Cu") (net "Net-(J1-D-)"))
 (segment (start 106.25 74.3275) (end 107.45 73.1275) (width 0.2) (layer "B.Cu") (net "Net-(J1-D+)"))
 (segment (start 105 78.1) (end 105 77.062244) (width 0.2) (layer "B.Cu") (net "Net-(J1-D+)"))
 (segment (start 106.25 75.812244) (end 106.25 74.3275) (width 0.2) (layer "B.Cu") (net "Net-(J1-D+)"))
 (segment (start 105 77.062244) (end 106.25 75.812244) (width 0.2) (layer "B.Cu") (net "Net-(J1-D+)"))
 (segment (start 105.95 78.1) (end 105.95 78.453052) (width 0.2) (layer "B.Cu") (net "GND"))
 (segment (start 103.8 78.203052) (end 103.8 74.2775) (width 0.2) (layer "B.Cu") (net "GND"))
 (segment (start 103.8 74.2775) (end 104.95 73.1275) (width 0.2) (layer "B.Cu") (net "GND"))
 (segment (start 105.340552 79.0625) (end 104.659448 79.0625) (width 0.2) (layer "B.Cu") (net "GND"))
 (segment (start 105.95 78.453052) (end 105.340552 79.0625) (width 0.2) (layer "B.Cu") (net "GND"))
 (segment (start 104.659448 79.0625) (end 103.8 78.203052) (width 0.2) (layer "B.Cu") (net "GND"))
 (segment (start 106.9 80.375) (end 108.575 80.375) (width 0.2) (layer "B.Cu") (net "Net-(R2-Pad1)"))
 (segment (start 108.575 80.375) (end 108.75 80.2) (width 0.2) (layer "B.Cu") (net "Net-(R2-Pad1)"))
 (segment (start 108.75 82.2) (end 108.75 83) (width 0.2) (layer "B.Cu") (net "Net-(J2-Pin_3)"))
 (segment (start 108.75 83) (end 107.15 84.6) (width 0.2) (layer "B.Cu") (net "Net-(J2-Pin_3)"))
 (segment (start 103.425 80.375) (end 103.25 80.2) (width 0.2) (layer "B.Cu") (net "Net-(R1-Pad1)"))
 (segment (start 105 80.375) (end 103.425 80.375) (width 0.2) (layer "B.Cu") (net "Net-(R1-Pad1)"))
 (segment (start 103.25 82.2) (end 103.25 82.7) (width 0.2) (layer "B.Cu") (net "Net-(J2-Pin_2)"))
 (segment (start 103.25 82.7) (end 105.15 84.6) (width 0.2) (layer "B.Cu") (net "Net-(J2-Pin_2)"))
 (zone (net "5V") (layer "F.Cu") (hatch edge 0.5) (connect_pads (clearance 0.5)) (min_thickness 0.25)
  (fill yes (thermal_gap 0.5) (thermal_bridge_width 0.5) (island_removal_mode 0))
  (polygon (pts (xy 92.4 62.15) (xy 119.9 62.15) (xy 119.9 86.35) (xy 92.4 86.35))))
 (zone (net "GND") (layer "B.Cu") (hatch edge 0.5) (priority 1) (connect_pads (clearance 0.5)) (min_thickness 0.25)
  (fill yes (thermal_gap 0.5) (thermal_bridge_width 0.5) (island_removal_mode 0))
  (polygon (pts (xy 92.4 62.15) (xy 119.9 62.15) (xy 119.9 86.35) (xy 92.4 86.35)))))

